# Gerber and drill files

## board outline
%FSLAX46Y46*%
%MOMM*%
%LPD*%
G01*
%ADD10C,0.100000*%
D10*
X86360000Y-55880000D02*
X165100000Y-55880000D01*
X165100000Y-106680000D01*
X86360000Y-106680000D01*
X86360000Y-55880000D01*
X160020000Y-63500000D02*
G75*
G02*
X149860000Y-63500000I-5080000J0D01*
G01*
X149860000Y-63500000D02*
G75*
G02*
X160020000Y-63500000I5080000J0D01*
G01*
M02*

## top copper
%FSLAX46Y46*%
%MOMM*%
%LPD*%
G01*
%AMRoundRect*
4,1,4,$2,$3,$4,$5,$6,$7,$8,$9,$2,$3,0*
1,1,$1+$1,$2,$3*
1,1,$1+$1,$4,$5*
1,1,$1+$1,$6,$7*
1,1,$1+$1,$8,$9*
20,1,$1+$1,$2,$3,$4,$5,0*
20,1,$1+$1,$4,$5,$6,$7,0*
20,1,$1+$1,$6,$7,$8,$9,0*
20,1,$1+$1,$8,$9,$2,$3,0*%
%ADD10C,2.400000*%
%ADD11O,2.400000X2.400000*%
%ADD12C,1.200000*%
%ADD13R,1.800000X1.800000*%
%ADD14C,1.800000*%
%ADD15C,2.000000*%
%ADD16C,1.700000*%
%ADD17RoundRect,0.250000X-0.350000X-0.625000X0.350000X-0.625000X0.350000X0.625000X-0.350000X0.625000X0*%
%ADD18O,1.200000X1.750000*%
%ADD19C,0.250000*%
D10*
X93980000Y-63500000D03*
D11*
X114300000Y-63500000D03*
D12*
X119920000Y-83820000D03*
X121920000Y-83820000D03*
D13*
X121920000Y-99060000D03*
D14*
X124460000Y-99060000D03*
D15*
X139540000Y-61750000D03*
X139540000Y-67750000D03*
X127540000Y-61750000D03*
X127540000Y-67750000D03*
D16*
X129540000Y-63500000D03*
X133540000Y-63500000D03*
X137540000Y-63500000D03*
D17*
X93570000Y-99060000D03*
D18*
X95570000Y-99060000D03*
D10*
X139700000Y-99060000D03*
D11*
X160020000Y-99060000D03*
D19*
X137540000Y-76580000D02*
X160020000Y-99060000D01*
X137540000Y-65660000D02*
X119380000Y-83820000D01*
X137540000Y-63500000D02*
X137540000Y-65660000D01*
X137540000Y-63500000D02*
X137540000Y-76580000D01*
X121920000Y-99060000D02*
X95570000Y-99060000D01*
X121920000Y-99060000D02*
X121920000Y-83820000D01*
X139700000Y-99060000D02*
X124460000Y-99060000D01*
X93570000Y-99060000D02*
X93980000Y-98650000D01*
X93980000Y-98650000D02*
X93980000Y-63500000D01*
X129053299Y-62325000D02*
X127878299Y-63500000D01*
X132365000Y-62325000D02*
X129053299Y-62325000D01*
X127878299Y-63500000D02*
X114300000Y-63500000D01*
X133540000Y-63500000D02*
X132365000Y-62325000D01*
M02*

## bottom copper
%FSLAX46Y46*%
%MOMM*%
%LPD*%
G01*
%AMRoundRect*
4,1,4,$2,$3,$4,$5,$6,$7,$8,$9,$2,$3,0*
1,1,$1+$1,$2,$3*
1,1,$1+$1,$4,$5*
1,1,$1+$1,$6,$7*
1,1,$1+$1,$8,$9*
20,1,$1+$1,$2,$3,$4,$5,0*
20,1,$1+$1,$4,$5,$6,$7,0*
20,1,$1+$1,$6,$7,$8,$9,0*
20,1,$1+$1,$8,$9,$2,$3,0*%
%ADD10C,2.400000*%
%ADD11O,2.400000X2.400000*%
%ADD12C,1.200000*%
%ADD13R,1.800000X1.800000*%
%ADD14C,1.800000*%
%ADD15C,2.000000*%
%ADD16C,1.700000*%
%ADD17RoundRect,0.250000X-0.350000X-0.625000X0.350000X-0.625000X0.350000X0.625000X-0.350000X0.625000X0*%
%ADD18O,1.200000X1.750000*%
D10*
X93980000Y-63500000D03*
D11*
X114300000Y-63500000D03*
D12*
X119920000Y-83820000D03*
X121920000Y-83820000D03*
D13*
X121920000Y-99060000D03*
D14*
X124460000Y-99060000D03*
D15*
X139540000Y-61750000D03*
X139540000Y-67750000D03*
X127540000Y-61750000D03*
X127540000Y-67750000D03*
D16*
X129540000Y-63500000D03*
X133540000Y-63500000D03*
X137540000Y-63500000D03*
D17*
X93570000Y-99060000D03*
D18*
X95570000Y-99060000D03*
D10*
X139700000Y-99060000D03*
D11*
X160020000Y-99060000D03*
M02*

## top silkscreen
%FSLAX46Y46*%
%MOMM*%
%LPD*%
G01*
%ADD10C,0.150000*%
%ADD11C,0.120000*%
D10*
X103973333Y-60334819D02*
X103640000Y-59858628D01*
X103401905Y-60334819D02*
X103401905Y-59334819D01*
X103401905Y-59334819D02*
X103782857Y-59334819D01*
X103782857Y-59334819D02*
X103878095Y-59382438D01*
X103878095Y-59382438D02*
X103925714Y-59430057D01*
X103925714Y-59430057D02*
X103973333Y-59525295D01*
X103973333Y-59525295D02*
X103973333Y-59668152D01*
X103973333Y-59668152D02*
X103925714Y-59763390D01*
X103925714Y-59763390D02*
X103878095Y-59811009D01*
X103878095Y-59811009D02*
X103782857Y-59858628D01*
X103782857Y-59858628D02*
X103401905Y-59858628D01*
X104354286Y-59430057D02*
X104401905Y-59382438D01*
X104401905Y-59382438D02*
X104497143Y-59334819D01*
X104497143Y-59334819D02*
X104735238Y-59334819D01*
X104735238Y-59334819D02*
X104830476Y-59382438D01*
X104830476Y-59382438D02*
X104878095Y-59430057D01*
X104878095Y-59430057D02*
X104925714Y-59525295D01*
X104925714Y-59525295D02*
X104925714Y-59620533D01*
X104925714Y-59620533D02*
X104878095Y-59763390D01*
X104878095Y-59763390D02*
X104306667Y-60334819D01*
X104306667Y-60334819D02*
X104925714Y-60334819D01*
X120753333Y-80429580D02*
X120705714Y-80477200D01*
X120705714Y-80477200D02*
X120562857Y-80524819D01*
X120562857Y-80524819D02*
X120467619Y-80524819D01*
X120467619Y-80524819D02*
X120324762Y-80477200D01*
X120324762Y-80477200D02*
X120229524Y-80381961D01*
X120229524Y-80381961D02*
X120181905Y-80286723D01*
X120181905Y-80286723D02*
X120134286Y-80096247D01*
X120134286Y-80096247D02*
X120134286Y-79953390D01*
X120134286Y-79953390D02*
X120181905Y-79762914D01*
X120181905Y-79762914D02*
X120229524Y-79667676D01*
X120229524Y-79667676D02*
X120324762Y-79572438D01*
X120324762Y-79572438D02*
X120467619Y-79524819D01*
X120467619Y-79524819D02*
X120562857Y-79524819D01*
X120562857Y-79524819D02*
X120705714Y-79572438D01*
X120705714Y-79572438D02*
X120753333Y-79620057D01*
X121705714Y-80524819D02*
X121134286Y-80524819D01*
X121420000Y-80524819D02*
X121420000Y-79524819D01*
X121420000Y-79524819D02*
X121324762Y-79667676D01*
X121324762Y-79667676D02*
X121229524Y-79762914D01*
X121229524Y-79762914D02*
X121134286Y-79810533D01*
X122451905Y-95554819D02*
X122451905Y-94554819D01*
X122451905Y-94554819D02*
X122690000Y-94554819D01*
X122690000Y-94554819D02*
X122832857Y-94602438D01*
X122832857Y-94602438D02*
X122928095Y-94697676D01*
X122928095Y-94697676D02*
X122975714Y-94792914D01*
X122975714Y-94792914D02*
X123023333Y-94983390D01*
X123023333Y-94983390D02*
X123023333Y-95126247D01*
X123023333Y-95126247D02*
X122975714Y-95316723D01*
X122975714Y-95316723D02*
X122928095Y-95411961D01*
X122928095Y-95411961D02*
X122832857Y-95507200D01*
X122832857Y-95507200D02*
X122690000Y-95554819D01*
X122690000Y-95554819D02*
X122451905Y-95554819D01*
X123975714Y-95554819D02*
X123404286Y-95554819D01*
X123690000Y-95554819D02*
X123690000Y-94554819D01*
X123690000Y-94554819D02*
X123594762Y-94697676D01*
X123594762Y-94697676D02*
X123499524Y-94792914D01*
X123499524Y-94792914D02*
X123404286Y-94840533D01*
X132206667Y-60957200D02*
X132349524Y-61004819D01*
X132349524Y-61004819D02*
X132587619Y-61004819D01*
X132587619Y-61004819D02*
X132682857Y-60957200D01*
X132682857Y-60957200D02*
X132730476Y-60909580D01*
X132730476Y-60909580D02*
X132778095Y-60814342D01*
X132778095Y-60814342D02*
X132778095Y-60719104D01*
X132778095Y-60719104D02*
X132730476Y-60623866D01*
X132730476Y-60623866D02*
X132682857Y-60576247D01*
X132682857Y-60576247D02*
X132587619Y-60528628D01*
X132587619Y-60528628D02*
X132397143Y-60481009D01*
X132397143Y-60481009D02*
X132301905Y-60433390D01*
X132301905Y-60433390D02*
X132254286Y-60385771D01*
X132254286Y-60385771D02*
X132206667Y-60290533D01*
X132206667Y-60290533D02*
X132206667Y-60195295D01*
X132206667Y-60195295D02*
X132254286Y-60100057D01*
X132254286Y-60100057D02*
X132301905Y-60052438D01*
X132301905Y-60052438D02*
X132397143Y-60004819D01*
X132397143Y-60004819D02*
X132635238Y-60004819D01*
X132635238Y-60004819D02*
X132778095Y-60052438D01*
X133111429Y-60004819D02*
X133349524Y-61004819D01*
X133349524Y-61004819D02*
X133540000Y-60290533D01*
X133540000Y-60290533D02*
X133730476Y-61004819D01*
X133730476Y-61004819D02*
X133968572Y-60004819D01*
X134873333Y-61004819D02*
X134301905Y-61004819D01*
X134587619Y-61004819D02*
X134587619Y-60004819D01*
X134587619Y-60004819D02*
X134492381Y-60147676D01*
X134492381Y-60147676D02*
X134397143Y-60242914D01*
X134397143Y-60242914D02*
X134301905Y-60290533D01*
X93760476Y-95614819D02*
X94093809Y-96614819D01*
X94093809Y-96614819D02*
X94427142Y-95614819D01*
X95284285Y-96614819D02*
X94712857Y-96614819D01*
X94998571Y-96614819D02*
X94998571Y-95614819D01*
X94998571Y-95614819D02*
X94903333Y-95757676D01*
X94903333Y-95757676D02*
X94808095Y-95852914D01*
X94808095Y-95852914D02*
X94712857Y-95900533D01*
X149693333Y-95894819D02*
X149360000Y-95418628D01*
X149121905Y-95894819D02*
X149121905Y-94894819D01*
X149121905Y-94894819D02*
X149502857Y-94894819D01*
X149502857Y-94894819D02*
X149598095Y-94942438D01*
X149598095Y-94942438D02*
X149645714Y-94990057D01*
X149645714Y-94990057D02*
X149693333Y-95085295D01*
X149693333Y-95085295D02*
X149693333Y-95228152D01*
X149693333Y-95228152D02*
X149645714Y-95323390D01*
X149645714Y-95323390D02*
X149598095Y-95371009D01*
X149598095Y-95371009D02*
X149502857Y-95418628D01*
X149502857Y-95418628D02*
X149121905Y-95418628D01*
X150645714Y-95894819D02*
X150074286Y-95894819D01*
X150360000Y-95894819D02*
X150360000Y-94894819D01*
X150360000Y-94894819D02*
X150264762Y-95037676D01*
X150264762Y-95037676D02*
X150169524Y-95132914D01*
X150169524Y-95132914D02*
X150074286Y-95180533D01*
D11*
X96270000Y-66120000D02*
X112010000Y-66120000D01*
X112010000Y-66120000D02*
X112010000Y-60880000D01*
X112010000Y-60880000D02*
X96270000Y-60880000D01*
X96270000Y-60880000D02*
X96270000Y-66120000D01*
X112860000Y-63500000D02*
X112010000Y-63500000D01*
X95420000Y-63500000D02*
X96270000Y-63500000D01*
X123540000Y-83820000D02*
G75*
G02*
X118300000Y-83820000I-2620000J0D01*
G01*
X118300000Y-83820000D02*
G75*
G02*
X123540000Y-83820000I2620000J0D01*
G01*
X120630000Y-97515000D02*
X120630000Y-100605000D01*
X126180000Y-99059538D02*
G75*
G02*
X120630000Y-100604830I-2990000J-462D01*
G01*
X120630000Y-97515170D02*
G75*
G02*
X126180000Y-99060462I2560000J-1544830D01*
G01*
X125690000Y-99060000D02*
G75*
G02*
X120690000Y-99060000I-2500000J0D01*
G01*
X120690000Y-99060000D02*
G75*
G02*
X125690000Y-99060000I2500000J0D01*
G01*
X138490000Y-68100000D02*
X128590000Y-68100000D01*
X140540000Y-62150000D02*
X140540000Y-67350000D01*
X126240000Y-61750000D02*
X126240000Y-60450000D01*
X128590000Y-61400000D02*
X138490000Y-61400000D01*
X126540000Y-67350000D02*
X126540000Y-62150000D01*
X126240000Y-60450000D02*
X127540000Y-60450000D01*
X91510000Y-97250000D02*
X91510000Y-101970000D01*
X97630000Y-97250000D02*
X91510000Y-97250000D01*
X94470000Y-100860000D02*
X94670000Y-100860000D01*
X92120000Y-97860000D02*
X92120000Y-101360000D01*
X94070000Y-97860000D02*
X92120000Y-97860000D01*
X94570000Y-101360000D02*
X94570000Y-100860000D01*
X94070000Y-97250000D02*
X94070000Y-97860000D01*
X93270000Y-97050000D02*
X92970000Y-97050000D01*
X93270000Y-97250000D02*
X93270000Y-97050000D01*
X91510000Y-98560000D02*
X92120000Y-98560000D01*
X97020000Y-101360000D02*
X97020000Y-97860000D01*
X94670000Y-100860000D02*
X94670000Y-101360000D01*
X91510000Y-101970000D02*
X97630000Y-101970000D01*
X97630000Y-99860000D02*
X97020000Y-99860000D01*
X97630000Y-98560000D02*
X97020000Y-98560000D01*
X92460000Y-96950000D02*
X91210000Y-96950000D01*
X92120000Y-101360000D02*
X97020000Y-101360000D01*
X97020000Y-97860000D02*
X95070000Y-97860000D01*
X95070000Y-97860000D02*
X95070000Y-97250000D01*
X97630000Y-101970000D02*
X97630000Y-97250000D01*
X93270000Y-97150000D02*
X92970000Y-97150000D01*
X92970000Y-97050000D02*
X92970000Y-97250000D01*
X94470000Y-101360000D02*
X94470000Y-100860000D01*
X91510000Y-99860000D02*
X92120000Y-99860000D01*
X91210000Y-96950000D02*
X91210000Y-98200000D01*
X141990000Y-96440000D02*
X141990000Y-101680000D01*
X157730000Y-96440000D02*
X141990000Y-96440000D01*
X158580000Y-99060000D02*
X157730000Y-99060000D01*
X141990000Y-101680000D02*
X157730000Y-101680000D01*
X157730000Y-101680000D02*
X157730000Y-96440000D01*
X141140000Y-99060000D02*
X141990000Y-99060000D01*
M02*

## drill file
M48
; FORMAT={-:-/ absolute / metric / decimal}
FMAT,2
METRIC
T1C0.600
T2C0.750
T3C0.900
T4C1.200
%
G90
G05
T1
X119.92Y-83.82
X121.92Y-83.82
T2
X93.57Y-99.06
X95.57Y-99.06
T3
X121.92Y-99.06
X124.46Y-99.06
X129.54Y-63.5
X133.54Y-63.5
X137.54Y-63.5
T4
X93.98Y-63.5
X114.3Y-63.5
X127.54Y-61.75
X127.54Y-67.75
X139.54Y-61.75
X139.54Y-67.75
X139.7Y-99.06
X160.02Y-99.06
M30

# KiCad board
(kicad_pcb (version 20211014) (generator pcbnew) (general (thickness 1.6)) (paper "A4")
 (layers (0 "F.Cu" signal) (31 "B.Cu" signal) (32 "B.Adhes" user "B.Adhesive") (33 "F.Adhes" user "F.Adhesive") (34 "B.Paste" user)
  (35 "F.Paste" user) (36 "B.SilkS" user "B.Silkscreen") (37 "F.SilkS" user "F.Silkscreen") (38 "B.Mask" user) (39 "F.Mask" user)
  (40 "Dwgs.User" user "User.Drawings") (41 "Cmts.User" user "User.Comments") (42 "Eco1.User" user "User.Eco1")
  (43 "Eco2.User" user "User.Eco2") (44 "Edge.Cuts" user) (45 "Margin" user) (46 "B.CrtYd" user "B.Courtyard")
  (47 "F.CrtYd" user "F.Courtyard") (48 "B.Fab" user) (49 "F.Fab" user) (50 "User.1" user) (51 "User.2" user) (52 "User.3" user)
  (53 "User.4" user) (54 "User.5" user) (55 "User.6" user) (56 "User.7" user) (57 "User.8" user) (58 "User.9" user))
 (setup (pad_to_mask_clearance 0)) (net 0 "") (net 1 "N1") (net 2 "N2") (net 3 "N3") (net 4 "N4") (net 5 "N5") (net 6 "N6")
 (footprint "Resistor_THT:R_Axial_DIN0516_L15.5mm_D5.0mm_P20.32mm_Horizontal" (layer "F.Cu") (at 93.98 63.5)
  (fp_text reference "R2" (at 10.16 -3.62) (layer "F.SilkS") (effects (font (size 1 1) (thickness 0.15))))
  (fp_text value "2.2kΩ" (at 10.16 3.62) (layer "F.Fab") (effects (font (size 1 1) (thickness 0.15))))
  (fp_line (start 2.29 2.62) (end 18.03 2.62) (layer "F.SilkS") (width 0.12))
  (fp_line (start 18.03 2.62) (end 18.03 -2.62) (layer "F.SilkS") (width 0.12))
  (fp_line (start 18.03 -2.62) (end 2.29 -2.62) (layer "F.SilkS") (width 0.12))
  (fp_line (start 2.29 -2.62) (end 2.29 2.62) (layer "F.SilkS") (width 0.12))
  (fp_line (start 18.88 0) (end 18.03 0) (layer "F.SilkS") (width 0.12))
  (fp_line (start 1.44 0) (end 2.29 0) (layer "F.SilkS") (width 0.12))
  (pad "1" thru_hole circle (at 0 0) (size 2.4 2.4) (drill 1.2) (layers *.Cu *.Mask) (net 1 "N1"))
  (pad "2" thru_hole oval (at 20.32 0) (size 2.4 2.4) (drill 1.2) (layers *.Cu *.Mask) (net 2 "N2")))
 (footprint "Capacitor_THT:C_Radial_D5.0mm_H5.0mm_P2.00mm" (layer "F.Cu") (at 119.92 83.82)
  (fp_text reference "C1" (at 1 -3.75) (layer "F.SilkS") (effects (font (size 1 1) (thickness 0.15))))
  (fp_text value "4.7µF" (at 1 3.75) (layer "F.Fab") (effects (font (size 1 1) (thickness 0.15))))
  (fp_circle (center 1 0) (end 3.62 0) (layer "F.SilkS") (width 0.12) (fill none))
  (pad "1" thru_hole circle (at 0 0) (size 1.2 1.2) (drill 0.6) (layers *.Cu *.Mask) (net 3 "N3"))
  (pad "2" thru_hole circle (at 2 0) (size 1.2 1.2) (drill 0.6) (layers *.Cu *.Mask) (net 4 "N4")))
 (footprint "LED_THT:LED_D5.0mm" (layer "F.Cu") (at 121.92 99.06)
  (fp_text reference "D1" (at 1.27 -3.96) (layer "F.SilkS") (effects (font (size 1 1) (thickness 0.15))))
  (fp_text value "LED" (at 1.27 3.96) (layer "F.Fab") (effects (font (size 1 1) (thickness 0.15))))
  (fp_line (start -1.29 -1.545) (end -1.29 1.545) (layer "F.SilkS") (width 0.12))
  (fp_arc (start 4.26 -0.000462) (mid 2.072002 2.880433) (end -1.29 1.54483) (layer "F.SilkS") (width 0.12))
  (fp_arc (start -1.29 -1.54483) (mid 2.072002 -2.880433) (end 4.26 0.000462) (layer "F.SilkS") (width 0.12))
  (fp_circle (center 1.27 0) (end 3.77 0) (layer "F.SilkS") (width 0.12) (fill none))
  (pad "1" thru_hole rect (at 0 0) (size 1.8 1.8) (drill 0.9) (layers *.Cu *.Mask) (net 4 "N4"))
  (pad "2" thru_hole circle (at 2.54 0) (size 1.8 1.8) (drill 0.9) (layers *.Cu *.Mask) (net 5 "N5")))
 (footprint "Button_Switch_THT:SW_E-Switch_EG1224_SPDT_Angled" (layer "F.Cu") (at 129.54 63.5)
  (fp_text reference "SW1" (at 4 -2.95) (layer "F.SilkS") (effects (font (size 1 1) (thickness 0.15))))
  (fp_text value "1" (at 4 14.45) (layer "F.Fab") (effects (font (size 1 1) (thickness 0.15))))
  (fp_line (start 8.95 4.6) (end -0.95 4.6) (layer "F.SilkS") (width 0.12))
  (fp_line (start 11 -1.35) (end 11 3.85) (layer "F.SilkS") (width 0.12))
  (fp_line (start -3.3 -1.75) (end -3.3 -3.05) (layer "F.SilkS") (width 0.12))
  (fp_line (start -0.95 -2.1) (end 8.95 -2.1) (layer "F.SilkS") (width 0.12))
  (fp_line (start -3 3.85) (end -3 -1.35) (layer "F.SilkS") (width 0.12))
  (fp_line (start -3.3 -3.05) (end -2 -3.05) (layer "F.SilkS") (width 0.12))
  (pad "" thru_hole circle (at 10 -1.75) (size 2 2) (drill 1.2) (layers *.Cu *.Mask))
  (pad "" thru_hole circle (at 10 4.25) (size 2 2) (drill 1.2) (layers *.Cu *.Mask))
  (pad "" thru_hole circle (at -2 -1.75) (size 2 2) (drill 1.2) (layers *.Cu *.Mask))
  (pad "" thru_hole circle (at -2 4.25) (size 2 2) (drill 1.2) (layers *.Cu *.Mask))
  (pad "1" thru_hole circle (at 0 0) (size 1.7 1.7) (drill 0.9) (layers *.Cu *.Mask) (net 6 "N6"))
  (pad "2" thru_hole circle (at 4 0) (size 1.7 1.7) (drill 0.9) (layers *.Cu *.Mask) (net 2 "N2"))
  (pad "3" thru_hole circle (at 8 0) (size 1.7 1.7) (drill 0.9) (layers *.Cu *.Mask) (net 3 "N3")))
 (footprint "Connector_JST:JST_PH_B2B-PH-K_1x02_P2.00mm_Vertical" (layer "F.Cu") (at 93.57 99.06)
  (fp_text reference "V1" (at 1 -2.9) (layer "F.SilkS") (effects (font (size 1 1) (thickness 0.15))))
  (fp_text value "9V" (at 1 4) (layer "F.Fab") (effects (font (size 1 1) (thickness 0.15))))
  (fp_line (start -2.06 -1.81) (end -2.06 2.91) (layer "F.SilkS") (width 0.12))
  (fp_line (start 4.06 -1.81) (end -2.06 -1.81) (layer "F.SilkS") (width 0.12))
  (fp_line (start 0.9 1.8) (end 1.1 1.8) (layer "F.SilkS") (width 0.12))
  (fp_line (start -1.45 -1.2) (end -1.45 2.3) (layer "F.SilkS") (width 0.12))
  (fp_line (start 0.5 -1.2) (end -1.45 -1.2) (layer "F.SilkS") (width 0.12))
  (fp_line (start 1 2.3) (end 1 1.8) (layer "F.SilkS") (width 0.12))
  (fp_line (start 0.5 -1.81) (end 0.5 -1.2) (layer "F.SilkS") (width 0.12))
  (fp_line (start -0.3 -2.01) (end -0.6 -2.01) (layer "F.SilkS") (width 0.12))
  (fp_line (start -0.3 -1.81) (end -0.3 -2.01) (layer "F.SilkS") (width 0.12))
  (fp_line (start -2.06 -0.5) (end -1.45 -0.5) (layer "F.SilkS") (width 0.12))
  (fp_line (start 3.45 2.3) (end 3.45 -1.2) (layer "F.SilkS") (width 0.12))
  (fp_line (start 1.1 1.8) (end 1.1 2.3) (layer "F.SilkS") (width 0.12))
  (fp_line (start -2.06 2.91) (end 4.06 2.91) (layer "F.SilkS") (width 0.12))
  (fp_line (start 4.06 0.8) (end 3.45 0.8) (layer "F.SilkS") (width 0.12))
  (fp_line (start 4.06 -0.5) (end 3.45 -0.5) (layer "F.SilkS") (width 0.12))
  (fp_line (start -1.11 -2.11) (end -2.36 -2.11) (layer "F.SilkS") (width 0.12))
  (fp_line (start -1.45 2.3) (end 3.45 2.3) (layer "F.SilkS") (width 0.12))
  (fp_line (start 3.45 -1.2) (end 1.5 -1.2) (layer "F.SilkS") (width 0.12))
  (fp_line (start 1.5 -1.2) (end 1.5 -1.81) (layer "F.SilkS") (width 0.12))
  (fp_line (start 4.06 2.91) (end 4.06 -1.81) (layer "F.SilkS") (width 0.12))
  (fp_line (start -0.3 -1.91) (end -0.6 -1.91) (layer "F.SilkS") (width 0.12))
  (fp_line (start -0.6 -2.01) (end -0.6 -1.81) (layer "F.SilkS") (width 0.12))
  (fp_line (start 0.9 2.3) (end 0.9 1.8) (layer "F.SilkS") (width 0.12))
  (fp_line (start -2.06 0.8) (end -1.45 0.8) (layer "F.SilkS") (width 0.12))
  (fp_line (start -2.36 -2.11) (end -2.36 -0.86) (layer "F.SilkS") (width 0.12))
  (pad "1" thru_hole roundrect (at 0 0) (size 1.2 1.75) (drill 0.75) (layers *.Cu *.Mask) (roundrect_rratio 0.208333) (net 1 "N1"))
  (pad "2" thru_hole oval (at 2 0) (size 1.2 1.75) (drill 0.75) (layers *.Cu *.Mask) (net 4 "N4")))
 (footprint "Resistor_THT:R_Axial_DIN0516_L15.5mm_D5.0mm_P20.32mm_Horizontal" (layer "F.Cu") (at 139.7 99.06)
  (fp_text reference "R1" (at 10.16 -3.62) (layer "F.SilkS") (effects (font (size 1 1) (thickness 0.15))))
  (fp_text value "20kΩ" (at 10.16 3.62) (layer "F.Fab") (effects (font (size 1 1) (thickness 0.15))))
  (fp_line (start 2.29 -2.62) (end 2.29 2.62) (layer "F.SilkS") (width 0.12))
  (fp_line (start 18.03 -2.62) (end 2.29 -2.62) (layer "F.SilkS") (width 0.12))
  (fp_line (start 18.88 0) (end 18.03 0) (layer "F.SilkS") (width 0.12))
  (fp_line (start 2.29 2.62) (end 18.03 2.62) (layer "F.SilkS") (width 0.12))
  (fp_line (start 18.03 2.62) (end 18.03 -2.62) (layer "F.SilkS") (width 0.12))
  (fp_line (start 1.44 0) (end 2.29 0) (layer "F.SilkS") (width 0.12))
  (pad "1" thru_hole circle (at 0 0) (size 2.4 2.4) (drill 1.2) (layers *.Cu *.Mask) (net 5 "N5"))
  (pad "2" thru_hole oval (at 20.32 0) (size 2.4 2.4) (drill 1.2) (layers *.Cu *.Mask) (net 3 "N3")))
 (gr_rect (start 86.36 55.88) (end 165.1 106.68) (layer "Edge.Cuts") (width 0.1) (fill none))
 (gr_circle (center 154.94 63.5) (end 160.02 63.5) (layer "Edge.Cuts") (width 0.1) (fill none))
 (gr_rect (start 165.1 81.28) (end 165.1 81.28) (layer "Edge.Cuts") (width 0.1) (fill none))
 (segment (start 137.54 76.58) (end 160.02 99.06) (width 0.25) (layer "F.Cu") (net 3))
 (segment (start 137.54 65.66) (end 119.38 83.82) (width 0.25) (layer "F.Cu") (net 3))
 (segment (start 137.54 63.5) (end 137.54 65.66) (width 0.25) (layer "F.Cu") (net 3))
 (segment (start 137.54 63.5) (end 137.54 76.58) (width 0.25) (layer "F.Cu") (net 3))
 (segment (start 121.92 99.06) (end 95.57 99.06) (width 0.25) (layer "F.Cu") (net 4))
 (segment (start 121.92 99.06) (end 121.92 83.82) (width 0.25) (layer "F.Cu") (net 4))
 (segment (start 139.7 99.06) (end 124.46 99.06) (width 0.25) (layer "F.Cu") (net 5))
 (segment (start 93.57 99.06) (end 93.98 98.65) (width 0.25) (layer "F.Cu") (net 1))
 (segment (start 93.98 98.65) (end 93.98 63.5) (width 0.25) (layer "F.Cu") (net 1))
 (segment (start 129.053299 62.325) (end 127.878299 63.5) (width 0.25) (layer "F.Cu") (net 2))
 (segment (start 132.365 62.325) (end 129.053299 62.325) (width 0.25) (layer "F.Cu") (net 2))
 (segment (start 127.878299 63.5) (end 114.3 63.5) (width 0.25) (layer "F.Cu") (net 2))
 (segment (start 133.54 63.5) (end 132.365 62.325) (width 0.25) (layer "F.Cu") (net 2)))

